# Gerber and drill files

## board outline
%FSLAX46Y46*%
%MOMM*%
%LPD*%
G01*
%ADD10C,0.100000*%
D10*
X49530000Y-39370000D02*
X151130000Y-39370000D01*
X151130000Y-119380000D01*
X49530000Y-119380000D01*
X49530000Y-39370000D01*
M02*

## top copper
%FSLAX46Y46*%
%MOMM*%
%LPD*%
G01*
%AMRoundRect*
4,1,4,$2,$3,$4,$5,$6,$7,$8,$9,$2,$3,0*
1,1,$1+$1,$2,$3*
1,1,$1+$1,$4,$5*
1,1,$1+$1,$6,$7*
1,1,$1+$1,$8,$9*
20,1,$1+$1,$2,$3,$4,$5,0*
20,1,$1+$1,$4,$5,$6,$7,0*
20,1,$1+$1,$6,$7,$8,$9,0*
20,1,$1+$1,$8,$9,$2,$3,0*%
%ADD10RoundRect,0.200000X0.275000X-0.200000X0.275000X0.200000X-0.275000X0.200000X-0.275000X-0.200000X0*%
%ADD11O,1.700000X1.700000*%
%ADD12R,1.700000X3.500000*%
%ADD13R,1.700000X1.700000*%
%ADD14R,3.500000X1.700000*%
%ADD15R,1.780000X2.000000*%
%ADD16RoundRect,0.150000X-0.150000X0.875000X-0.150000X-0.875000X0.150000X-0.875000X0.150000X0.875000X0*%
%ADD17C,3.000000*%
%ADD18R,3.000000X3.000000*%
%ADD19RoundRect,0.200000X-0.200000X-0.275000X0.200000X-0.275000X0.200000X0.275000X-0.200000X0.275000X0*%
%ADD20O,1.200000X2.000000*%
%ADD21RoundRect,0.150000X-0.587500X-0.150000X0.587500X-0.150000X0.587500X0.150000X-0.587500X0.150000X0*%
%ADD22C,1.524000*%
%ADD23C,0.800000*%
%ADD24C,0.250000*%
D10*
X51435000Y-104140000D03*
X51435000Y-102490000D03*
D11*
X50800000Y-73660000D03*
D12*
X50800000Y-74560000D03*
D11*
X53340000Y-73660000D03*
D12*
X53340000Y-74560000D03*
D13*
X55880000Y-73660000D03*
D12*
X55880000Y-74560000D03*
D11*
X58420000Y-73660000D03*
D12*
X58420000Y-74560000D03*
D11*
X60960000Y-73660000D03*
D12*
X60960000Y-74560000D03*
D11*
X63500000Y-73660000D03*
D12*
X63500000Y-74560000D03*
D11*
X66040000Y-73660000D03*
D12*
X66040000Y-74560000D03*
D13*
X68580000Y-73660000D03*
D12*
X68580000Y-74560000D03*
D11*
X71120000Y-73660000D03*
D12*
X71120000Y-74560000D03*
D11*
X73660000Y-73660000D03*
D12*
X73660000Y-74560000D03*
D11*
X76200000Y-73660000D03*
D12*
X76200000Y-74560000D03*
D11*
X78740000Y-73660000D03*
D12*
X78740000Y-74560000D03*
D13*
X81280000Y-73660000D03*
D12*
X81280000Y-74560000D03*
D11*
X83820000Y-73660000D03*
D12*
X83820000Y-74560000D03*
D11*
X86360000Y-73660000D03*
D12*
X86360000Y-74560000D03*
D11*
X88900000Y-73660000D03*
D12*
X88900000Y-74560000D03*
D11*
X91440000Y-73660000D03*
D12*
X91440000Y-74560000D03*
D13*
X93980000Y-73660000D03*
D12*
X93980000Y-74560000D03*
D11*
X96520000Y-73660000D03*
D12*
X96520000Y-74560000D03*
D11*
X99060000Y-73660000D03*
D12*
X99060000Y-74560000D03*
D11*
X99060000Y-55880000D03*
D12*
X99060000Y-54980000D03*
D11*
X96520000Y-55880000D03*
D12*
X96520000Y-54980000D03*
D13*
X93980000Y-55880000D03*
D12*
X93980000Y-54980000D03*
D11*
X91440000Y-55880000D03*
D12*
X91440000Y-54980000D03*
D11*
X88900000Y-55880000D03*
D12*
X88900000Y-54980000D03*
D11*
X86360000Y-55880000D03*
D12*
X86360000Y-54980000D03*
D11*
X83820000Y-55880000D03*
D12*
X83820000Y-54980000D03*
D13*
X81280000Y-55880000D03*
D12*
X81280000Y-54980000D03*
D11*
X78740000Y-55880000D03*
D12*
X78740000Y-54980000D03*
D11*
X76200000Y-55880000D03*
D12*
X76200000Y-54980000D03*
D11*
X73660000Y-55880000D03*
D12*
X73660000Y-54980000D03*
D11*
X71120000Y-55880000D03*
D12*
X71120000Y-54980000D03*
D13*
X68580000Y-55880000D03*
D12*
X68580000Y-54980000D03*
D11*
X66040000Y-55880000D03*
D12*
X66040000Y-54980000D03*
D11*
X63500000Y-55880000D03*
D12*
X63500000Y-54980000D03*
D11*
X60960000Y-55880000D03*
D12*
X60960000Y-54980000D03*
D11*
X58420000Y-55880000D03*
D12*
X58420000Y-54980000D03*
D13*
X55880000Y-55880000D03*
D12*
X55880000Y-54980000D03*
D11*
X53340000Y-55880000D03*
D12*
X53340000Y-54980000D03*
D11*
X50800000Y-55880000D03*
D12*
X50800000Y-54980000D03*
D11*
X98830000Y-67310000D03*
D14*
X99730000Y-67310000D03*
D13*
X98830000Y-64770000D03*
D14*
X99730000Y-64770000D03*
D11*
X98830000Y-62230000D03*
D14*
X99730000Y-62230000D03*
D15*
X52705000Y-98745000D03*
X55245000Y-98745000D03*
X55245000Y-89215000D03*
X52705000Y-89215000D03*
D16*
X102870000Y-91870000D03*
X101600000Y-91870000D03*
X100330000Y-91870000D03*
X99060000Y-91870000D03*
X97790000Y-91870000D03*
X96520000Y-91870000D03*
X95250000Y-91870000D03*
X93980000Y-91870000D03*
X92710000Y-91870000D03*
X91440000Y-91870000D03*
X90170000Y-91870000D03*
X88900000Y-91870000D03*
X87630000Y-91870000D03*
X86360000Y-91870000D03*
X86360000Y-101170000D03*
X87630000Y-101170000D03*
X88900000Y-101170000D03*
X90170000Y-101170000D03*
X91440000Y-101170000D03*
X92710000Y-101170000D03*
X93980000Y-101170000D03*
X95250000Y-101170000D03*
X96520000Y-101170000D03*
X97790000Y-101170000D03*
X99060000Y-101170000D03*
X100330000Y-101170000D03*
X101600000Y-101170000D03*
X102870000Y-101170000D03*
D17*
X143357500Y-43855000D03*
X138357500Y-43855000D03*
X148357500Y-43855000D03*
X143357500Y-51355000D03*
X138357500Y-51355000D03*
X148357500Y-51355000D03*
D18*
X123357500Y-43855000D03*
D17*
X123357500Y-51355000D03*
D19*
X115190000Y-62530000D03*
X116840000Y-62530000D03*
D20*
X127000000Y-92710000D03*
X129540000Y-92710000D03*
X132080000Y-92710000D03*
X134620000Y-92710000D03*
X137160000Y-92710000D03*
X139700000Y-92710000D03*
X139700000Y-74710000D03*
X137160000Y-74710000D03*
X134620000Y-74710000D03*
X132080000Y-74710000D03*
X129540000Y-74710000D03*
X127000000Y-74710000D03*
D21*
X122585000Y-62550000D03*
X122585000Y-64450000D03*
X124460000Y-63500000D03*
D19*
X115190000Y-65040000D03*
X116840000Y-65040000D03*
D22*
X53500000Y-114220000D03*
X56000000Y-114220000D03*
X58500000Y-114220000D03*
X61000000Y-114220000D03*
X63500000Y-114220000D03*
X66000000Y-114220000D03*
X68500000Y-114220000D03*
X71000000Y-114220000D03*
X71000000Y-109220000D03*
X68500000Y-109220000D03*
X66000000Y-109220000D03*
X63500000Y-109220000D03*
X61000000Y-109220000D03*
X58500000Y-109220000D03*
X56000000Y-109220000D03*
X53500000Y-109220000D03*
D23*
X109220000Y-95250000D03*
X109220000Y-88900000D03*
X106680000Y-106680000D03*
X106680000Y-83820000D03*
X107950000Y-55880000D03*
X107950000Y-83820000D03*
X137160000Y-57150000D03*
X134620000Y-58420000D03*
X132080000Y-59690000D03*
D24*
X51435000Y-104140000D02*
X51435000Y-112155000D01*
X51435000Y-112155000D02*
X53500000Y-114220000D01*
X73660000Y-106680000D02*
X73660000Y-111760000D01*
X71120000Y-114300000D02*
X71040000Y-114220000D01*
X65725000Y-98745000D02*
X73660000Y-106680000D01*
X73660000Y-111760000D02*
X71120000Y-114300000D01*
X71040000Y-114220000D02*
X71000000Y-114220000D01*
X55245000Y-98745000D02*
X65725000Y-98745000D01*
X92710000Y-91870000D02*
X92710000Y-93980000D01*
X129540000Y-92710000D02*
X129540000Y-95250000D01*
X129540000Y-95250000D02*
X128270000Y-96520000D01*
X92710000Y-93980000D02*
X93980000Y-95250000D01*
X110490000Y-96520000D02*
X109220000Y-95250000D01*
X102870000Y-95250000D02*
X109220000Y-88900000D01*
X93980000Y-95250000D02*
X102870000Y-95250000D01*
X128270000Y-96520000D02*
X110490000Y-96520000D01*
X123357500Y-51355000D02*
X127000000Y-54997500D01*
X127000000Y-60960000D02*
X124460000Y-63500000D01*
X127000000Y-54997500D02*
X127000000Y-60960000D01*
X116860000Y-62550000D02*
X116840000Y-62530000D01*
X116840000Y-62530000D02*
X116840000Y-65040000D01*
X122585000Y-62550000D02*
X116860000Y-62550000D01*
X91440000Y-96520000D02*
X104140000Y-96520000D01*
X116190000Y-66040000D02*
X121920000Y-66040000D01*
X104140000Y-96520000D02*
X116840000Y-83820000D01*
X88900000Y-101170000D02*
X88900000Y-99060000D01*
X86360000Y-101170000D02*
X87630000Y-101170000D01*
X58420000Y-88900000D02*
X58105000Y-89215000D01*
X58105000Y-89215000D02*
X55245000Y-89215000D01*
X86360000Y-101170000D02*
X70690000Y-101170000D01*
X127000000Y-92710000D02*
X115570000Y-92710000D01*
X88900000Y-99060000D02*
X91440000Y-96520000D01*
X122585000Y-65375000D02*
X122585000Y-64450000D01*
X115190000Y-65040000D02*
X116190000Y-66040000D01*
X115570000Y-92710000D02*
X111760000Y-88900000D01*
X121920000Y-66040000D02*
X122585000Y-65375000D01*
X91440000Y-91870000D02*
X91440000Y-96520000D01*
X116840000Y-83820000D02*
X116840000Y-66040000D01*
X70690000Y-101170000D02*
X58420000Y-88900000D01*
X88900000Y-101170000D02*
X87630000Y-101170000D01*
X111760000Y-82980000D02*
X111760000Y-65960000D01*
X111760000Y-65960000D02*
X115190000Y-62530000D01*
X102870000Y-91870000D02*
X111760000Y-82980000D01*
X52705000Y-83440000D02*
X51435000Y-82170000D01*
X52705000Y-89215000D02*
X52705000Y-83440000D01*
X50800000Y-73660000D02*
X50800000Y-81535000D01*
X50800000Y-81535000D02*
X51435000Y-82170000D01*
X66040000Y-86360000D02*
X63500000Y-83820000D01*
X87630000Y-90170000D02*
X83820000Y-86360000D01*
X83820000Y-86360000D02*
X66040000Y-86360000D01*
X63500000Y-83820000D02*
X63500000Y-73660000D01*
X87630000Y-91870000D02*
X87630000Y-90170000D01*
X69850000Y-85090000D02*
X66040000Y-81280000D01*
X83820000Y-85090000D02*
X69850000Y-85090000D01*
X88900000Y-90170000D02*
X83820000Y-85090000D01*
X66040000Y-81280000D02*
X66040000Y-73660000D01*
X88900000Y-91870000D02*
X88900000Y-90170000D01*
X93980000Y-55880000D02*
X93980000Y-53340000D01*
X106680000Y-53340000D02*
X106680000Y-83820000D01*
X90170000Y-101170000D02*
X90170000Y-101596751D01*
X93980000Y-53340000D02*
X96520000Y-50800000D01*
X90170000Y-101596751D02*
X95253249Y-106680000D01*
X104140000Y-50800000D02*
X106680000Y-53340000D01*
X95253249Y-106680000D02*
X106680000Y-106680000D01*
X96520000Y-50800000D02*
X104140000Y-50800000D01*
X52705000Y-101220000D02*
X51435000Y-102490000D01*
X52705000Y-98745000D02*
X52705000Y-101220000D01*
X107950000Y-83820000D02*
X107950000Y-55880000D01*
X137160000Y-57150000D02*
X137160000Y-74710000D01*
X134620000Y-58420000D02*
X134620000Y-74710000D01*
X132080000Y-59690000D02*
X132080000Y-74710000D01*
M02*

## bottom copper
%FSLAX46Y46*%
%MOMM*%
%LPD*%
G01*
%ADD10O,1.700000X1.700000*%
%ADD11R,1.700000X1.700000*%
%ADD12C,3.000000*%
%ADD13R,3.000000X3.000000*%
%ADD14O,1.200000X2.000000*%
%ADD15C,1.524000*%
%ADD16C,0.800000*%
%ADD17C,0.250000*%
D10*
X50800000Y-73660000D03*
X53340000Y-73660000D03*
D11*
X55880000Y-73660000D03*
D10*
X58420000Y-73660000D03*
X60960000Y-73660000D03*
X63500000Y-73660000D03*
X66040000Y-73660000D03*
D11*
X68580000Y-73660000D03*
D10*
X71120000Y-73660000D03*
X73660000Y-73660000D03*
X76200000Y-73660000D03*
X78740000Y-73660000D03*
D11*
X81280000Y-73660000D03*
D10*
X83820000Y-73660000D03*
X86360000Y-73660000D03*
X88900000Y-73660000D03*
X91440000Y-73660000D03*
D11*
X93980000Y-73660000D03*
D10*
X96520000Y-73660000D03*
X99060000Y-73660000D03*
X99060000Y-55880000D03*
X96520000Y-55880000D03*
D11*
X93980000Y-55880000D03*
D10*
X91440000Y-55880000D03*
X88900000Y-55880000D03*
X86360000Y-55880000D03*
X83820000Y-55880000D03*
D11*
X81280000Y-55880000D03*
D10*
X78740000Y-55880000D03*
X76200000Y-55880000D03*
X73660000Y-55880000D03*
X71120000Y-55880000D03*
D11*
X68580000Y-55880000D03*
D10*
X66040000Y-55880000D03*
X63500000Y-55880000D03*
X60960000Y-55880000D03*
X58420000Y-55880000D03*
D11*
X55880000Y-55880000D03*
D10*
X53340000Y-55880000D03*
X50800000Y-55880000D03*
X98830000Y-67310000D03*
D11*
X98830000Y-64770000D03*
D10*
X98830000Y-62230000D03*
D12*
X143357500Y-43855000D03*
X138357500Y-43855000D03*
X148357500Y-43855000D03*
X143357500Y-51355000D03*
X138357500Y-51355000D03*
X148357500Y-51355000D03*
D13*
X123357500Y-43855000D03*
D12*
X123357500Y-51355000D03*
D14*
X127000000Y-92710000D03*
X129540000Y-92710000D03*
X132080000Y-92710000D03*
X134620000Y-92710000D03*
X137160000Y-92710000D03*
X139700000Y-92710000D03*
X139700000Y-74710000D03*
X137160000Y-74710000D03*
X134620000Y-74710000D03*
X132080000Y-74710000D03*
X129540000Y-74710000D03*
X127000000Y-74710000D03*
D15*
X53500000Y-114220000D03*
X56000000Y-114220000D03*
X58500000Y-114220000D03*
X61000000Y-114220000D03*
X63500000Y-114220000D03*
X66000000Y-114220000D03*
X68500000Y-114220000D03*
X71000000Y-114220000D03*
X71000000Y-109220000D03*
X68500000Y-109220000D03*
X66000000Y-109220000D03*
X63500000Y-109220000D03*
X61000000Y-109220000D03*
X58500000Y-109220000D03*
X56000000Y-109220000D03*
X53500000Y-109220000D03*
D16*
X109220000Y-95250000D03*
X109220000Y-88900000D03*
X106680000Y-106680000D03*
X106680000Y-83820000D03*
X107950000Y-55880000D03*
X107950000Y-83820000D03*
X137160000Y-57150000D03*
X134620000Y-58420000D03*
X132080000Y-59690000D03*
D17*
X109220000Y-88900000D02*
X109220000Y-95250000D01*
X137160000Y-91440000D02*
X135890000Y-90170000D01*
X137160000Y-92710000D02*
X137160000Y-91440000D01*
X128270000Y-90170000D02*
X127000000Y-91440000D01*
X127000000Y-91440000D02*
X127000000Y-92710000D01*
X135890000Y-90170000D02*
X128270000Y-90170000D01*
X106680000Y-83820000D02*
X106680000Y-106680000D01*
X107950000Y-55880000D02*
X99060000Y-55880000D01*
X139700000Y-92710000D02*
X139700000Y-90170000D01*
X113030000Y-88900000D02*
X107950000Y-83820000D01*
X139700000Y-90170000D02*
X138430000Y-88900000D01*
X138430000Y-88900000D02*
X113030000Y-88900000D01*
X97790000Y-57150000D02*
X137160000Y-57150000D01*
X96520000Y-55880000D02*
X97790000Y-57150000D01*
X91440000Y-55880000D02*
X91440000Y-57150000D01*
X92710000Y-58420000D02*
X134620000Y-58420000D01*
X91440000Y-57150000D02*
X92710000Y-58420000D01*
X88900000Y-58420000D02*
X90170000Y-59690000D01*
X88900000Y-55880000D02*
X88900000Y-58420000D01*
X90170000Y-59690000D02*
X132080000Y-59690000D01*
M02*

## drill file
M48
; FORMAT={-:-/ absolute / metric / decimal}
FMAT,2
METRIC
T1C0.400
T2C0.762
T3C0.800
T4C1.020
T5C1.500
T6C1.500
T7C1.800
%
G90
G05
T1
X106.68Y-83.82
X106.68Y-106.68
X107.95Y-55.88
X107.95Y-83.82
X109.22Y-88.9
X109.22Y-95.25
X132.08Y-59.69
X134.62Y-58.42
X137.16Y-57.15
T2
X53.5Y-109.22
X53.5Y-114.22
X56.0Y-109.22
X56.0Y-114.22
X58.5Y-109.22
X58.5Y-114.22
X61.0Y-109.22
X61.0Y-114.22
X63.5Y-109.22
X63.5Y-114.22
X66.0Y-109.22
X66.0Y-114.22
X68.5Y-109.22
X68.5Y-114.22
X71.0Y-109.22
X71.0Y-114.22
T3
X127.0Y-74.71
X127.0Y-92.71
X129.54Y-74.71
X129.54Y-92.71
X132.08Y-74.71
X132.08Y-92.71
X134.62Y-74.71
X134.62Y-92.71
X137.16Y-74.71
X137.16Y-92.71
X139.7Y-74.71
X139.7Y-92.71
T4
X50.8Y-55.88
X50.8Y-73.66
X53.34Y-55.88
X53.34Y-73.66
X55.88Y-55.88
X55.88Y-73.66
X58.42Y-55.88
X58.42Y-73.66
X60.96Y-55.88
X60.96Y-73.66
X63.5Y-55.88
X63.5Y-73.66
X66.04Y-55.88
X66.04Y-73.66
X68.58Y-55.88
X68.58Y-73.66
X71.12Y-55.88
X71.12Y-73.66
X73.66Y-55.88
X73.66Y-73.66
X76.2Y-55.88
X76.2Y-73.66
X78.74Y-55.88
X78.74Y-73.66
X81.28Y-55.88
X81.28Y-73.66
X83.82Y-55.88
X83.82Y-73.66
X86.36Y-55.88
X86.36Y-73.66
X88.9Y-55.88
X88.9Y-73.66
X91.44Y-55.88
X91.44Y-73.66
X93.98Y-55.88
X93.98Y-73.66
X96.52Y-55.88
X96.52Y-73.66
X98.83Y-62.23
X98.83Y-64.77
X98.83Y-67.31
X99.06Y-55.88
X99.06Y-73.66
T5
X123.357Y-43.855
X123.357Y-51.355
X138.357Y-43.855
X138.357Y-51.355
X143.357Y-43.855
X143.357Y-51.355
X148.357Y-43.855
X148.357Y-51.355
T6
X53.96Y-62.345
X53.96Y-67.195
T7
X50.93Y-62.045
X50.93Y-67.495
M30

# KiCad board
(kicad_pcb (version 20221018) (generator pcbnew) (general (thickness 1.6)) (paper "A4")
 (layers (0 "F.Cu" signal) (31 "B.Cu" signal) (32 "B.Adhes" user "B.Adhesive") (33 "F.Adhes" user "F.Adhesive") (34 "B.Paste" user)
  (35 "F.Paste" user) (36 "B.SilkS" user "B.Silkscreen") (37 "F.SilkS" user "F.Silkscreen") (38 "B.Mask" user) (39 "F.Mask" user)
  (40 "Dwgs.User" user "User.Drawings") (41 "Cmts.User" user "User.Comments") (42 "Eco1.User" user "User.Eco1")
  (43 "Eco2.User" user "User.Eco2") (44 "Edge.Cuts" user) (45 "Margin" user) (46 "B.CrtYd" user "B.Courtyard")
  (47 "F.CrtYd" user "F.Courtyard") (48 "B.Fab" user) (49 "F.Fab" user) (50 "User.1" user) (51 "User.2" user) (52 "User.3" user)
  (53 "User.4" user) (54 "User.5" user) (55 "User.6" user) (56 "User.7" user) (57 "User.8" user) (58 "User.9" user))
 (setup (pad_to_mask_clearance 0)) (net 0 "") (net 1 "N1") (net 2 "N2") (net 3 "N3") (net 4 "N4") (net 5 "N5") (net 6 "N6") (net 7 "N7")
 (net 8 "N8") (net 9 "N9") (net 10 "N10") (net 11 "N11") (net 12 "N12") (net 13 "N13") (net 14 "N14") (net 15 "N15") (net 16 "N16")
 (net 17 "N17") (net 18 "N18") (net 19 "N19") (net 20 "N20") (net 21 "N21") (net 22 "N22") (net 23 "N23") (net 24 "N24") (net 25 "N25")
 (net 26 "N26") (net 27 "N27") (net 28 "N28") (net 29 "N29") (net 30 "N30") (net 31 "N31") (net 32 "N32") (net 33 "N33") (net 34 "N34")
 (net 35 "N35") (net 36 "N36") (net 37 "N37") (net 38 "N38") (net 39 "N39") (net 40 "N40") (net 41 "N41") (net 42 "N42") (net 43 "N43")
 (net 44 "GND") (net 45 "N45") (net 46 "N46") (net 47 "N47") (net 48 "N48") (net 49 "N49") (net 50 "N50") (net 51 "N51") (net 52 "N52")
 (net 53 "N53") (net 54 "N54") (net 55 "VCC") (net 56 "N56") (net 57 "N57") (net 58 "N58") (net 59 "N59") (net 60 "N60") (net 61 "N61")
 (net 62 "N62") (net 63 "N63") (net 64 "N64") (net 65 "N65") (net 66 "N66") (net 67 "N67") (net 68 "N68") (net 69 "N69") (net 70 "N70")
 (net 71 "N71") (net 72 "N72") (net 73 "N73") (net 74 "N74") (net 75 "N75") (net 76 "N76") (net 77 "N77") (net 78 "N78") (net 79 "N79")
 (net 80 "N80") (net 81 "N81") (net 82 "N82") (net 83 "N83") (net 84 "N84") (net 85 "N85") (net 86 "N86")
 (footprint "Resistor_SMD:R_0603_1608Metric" (layer "F.Cu") (at 51.435 103.315 90)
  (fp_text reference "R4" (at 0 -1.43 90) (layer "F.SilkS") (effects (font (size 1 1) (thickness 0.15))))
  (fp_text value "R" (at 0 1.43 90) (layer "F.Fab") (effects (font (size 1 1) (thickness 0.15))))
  (pad "1" smd roundrect (at -0.825 0 90) (size 0.8 0.95) (layers "F.Cu" "F.Paste" "F.Mask") (roundrect_rratio 0.25) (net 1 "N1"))
  (pad "2" smd roundrect (at 0.825 0 90) (size 0.8 0.95) (layers "F.Cu" "F.Paste" "F.Mask") (roundrect_rratio 0.25) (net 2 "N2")))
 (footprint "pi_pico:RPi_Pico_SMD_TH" (layer "F.Cu") (at 74.93 64.77 90)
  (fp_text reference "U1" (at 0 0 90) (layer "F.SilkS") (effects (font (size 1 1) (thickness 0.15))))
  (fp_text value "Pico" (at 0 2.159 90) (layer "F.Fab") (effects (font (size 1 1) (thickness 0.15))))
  (pad "" np_thru_hole oval (at -2.725 -24 90) (size 1.8 1.8) (drill 1.8) (layers "*.Cu" "*.Mask"))
  (pad "" np_thru_hole oval (at -2.425 -20.97 90) (size 1.5 1.5) (drill 1.5) (layers "*.Cu" "*.Mask"))
  (pad "" np_thru_hole oval (at 2.425 -20.97 90) (size 1.5 1.5) (drill 1.5) (layers "*.Cu" "*.Mask"))
  (pad "" np_thru_hole oval (at 2.725 -24 90) (size 1.8 1.8) (drill 1.8) (layers "*.Cu" "*.Mask"))
  (pad "1" thru_hole oval (at -8.89 -24.13 90) (size 1.7 1.7) (drill 1.02) (layers "*.Cu" "*.Mask") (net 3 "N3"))
  (pad "1" smd rect (at -8.89 -24.13 90) (size 3.5 1.7) (drill (offset -0.9 0)) (layers "F.Cu" "F.Mask") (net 3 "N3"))
  (pad "2" thru_hole oval (at -8.89 -21.59 90) (size 1.7 1.7) (drill 1.02) (layers "*.Cu" "*.Mask") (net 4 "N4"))
  (pad "2" smd rect (at -8.89 -21.59 90) (size 3.5 1.7) (drill (offset -0.9 0)) (layers "F.Cu" "F.Mask") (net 4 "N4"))
  (pad "3" thru_hole rect (at -8.89 -19.05 90) (size 1.7 1.7) (drill 1.02) (layers "*.Cu" "*.Mask") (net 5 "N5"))
  (pad "3" smd rect (at -8.89 -19.05 90) (size 3.5 1.7) (drill (offset -0.9 0)) (layers "F.Cu" "F.Mask") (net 5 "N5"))
  (pad "4" thru_hole oval (at -8.89 -16.51 90) (size 1.7 1.7) (drill 1.02) (layers "*.Cu" "*.Mask") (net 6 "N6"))
  (pad "4" smd rect (at -8.89 -16.51 90) (size 3.5 1.7) (drill (offset -0.9 0)) (layers "F.Cu" "F.Mask") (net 6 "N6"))
  (pad "5" thru_hole oval (at -8.89 -13.97 90) (size 1.7 1.7) (drill 1.02) (layers "*.Cu" "*.Mask") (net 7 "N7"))
  (pad "5" smd rect (at -8.89 -13.97 90) (size 3.5 1.7) (drill (offset -0.9 0)) (layers "F.Cu" "F.Mask") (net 7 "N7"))
  (pad "6" thru_hole oval (at -8.89 -11.43 90) (size 1.7 1.7) (drill 1.02) (layers "*.Cu" "*.Mask") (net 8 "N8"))
  (pad "6" smd rect (at -8.89 -11.43 90) (size 3.5 1.7) (drill (offset -0.9 0)) (layers "F.Cu" "F.Mask") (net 8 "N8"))
  (pad "7" thru_hole oval (at -8.89 -8.89 90) (size 1.7 1.7) (drill 1.02) (layers "*.Cu" "*.Mask") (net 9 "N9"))
  (pad "7" smd rect (at -8.89 -8.89 90) (size 3.5 1.7) (drill (offset -0.9 0)) (layers "F.Cu" "F.Mask") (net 9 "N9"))
  (pad "8" thru_hole rect (at -8.89 -6.35 90) (size 1.7 1.7) (drill 1.02) (layers "*.Cu" "*.Mask") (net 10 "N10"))
  (pad "8" smd rect (at -8.89 -6.35 90) (size 3.5 1.7) (drill (offset -0.9 0)) (layers "F.Cu" "F.Mask") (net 10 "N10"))
  (pad "9" thru_hole oval (at -8.89 -3.81 90) (size 1.7 1.7) (drill 1.02) (layers "*.Cu" "*.Mask") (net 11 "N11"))
  (pad "9" smd rect (at -8.89 -3.81 90) (size 3.5 1.7) (drill (offset -0.9 0)) (layers "F.Cu" "F.Mask") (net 11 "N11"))
  (pad "10" thru_hole oval (at -8.89 -1.27 90) (size 1.7 1.7) (drill 1.02) (layers "*.Cu" "*.Mask") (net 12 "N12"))
  (pad "10" smd rect (at -8.89 -1.27 90) (size 3.5 1.7) (drill (offset -0.9 0)) (layers "F.Cu" "F.Mask") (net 12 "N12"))
  (pad "11" thru_hole oval (at -8.89 1.27 90) (size 1.7 1.7) (drill 1.02) (layers "*.Cu" "*.Mask") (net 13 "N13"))
  (pad "11" smd rect (at -8.89 1.27 90) (size 3.5 1.7) (drill (offset -0.9 0)) (layers "F.Cu" "F.Mask") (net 13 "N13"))
  (pad "12" thru_hole oval (at -8.89 3.81 90) (size 1.7 1.7) (drill 1.02) (layers "*.Cu" "*.Mask") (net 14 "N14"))
  (pad "12" smd rect (at -8.89 3.81 90) (size 3.5 1.7) (drill (offset -0.9 0)) (layers "F.Cu" "F.Mask") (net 14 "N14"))
  (pad "13" thru_hole rect (at -8.89 6.35 90) (size 1.7 1.7) (drill 1.02) (layers "*.Cu" "*.Mask") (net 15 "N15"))
  (pad "13" smd rect (at -8.89 6.35 90) (size 3.5 1.7) (drill (offset -0.9 0)) (layers "F.Cu" "F.Mask") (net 15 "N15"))
  (pad "14" thru_hole oval (at -8.89 8.89 90) (size 1.7 1.7) (drill 1.02) (layers "*.Cu" "*.Mask") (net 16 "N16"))
  (pad "14" smd rect (at -8.89 8.89 90) (size 3.5 1.7) (drill (offset -0.9 0)) (layers "F.Cu" "F.Mask") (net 16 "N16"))
  (pad "15" thru_hole oval (at -8.89 11.43 90) (size 1.7 1.7) (drill 1.02) (layers "*.Cu" "*.Mask") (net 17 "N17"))
  (pad "15" smd rect (at -8.89 11.43 90) (size 3.5 1.7) (drill (offset -0.9 0)) (layers "F.Cu" "F.Mask") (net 17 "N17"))
  (pad "16" thru_hole oval (at -8.89 13.97 90) (size 1.7 1.7) (drill 1.02) (layers "*.Cu" "*.Mask") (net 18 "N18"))
  (pad "16" smd rect (at -8.89 13.97 90) (size 3.5 1.7) (drill (offset -0.9 0)) (layers "F.Cu" "F.Mask") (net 18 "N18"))
  (pad "17" thru_hole oval (at -8.89 16.51 90) (size 1.7 1.7) (drill 1.02) (layers "*.Cu" "*.Mask") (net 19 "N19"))
  (pad "17" smd rect (at -8.89 16.51 90) (size 3.5 1.7) (drill (offset -0.9 0)) (layers "F.Cu" "F.Mask") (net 19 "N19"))
  (pad "18" thru_hole rect (at -8.89 19.05 90) (size 1.7 1.7) (drill 1.02) (layers "*.Cu" "*.Mask") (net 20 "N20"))
  (pad "18" smd rect (at -8.89 19.05 90) (size 3.5 1.7) (drill (offset -0.9 0)) (layers "F.Cu" "F.Mask") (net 20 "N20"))
  (pad "19" thru_hole oval (at -8.89 21.59 90) (size 1.7 1.7) (drill 1.02) (layers "*.Cu" "*.Mask") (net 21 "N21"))
  (pad "19" smd rect (at -8.89 21.59 90) (size 3.5 1.7) (drill (offset -0.9 0)) (layers "F.Cu" "F.Mask") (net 21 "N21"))
  (pad "20" thru_hole oval (at -8.89 24.13 90) (size 1.7 1.7) (drill 1.02) (layers "*.Cu" "*.Mask") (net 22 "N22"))
  (pad "20" smd rect (at -8.89 24.13 90) (size 3.5 1.7) (drill (offset -0.9 0)) (layers "F.Cu" "F.Mask") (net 22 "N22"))
  (pad "21" thru_hole oval (at 8.89 24.13 90) (size 1.7 1.7) (drill 1.02) (layers "*.Cu" "*.Mask") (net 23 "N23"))
  (pad "21" smd rect (at 8.89 24.13 90) (size 3.5 1.7) (drill (offset 0.9 0)) (layers "F.Cu" "F.Mask") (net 23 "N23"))
  (pad "22" thru_hole oval (at 8.89 21.59 90) (size 1.7 1.7) (drill 1.02) (layers "*.Cu" "*.Mask") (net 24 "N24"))
  (pad "22" smd rect (at 8.89 21.59 90) (size 3.5 1.7) (drill (offset 0.9 0)) (layers "F.Cu" "F.Mask") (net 24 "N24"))
  (pad "23" thru_hole rect (at 8.89 19.05 90) (size 1.7 1.7) (drill 1.02) (layers "*.Cu" "*.Mask") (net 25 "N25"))
  (pad "23" smd rect (at 8.89 19.05 90) (size 3.5 1.7) (drill (offset 0.9 0)) (layers "F.Cu" "F.Mask") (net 25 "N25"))
  (pad "24" thru_hole oval (at 8.89 16.51 90) (size 1.7 1.7) (drill 1.02) (layers "*.Cu" "*.Mask") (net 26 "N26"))
  (pad "24" smd rect (at 8.89 16.51 90) (size 3.5 1.7) (drill (offset 0.9 0)) (layers "F.Cu" "F.Mask") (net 26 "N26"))
  (pad "25" thru_hole oval (at 8.89 13.97 90) (size 1.7 1.7) (drill 1.02) (layers "*.Cu" "*.Mask") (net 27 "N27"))
  (pad "25" smd rect (at 8.89 13.97 90) (size 3.5 1.7) (drill (offset 0.9 0)) (layers "F.Cu" "F.Mask") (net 27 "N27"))
  (pad "26" thru_hole oval (at 8.89 11.43 90) (size 1.7 1.7) (drill 1.02) (layers "*.Cu" "*.Mask") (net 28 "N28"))
  (pad "26" smd rect (at 8.89 11.43 90) (size 3.5 1.7) (drill (offset 0.9 0)) (layers "F.Cu" "F.Mask") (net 28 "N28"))
  (pad "27" thru_hole oval (at 8.89 8.89 90) (size 1.7 1.7) (drill 1.02) (layers "*.Cu" "*.Mask") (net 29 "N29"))
  (pad "27" smd rect (at 8.89 8.89 90) (size 3.5 1.7) (drill (offset 0.9 0)) (layers "F.Cu" "F.Mask") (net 29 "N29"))
  (pad "28" thru_hole rect (at 8.89 6.35 90) (size 1.7 1.7) (drill 1.02) (layers "*.Cu" "*.Mask") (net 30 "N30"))
  (pad "28" smd rect (at 8.89 6.35 90) (size 3.5 1.7) (drill (offset 0.9 0)) (layers "F.Cu" "F.Mask") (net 30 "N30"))
  (pad "29" thru_hole oval (at 8.89 3.81 90) (size 1.7 1.7) (drill 1.02) (layers "*.Cu" "*.Mask") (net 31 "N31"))
  (pad "29" smd rect (at 8.89 3.81 90) (size 3.5 1.7) (drill (offset 0.9 0)) (layers "F.Cu" "F.Mask") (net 31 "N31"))
  (pad "30" thru_hole oval (at 8.89 1.27 90) (size 1.7 1.7) (drill 1.02) (layers "*.Cu" "*.Mask") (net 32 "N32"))
  (pad "30" smd rect (at 8.89 1.27 90) (size 3.5 1.7) (drill (offset 0.9 0)) (layers "F.Cu" "F.Mask") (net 32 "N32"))
  (pad "31" thru_hole oval (at 8.89 -1.27 90) (size 1.7 1.7) (drill 1.02) (layers "*.Cu" "*.Mask") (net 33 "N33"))
  (pad "31" smd rect (at 8.89 -1.27 90) (size 3.5 1.7) (drill (offset 0.9 0)) (layers "F.Cu" "F.Mask") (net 33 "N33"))
  (pad "32" thru_hole oval (at 8.89 -3.81 90) (size 1.7 1.7) (drill 1.02) (layers "*.Cu" "*.Mask") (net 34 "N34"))
  (pad "32" smd rect (at 8.89 -3.81 90) (size 3.5 1.7) (drill (offset 0.9 0)) (layers "F.Cu" "F.Mask") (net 34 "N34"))
  (pad "33" thru_hole rect (at 8.89 -6.35 90) (size 1.7 1.7) (drill 1.02) (layers "*.Cu" "*.Mask") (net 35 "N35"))
  (pad "33" smd rect (at 8.89 -6.35 90) (size 3.5 1.7) (drill (offset 0.9 0)) (layers "F.Cu" "F.Mask") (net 35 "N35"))
  (pad "34" thru_hole oval (at 8.89 -8.89 90) (size 1.7 1.7) (drill 1.02) (layers "*.Cu" "*.Mask") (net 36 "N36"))
  (pad "34" smd rect (at 8.89 -8.89 90) (size 3.5 1.7) (drill (offset 0.9 0)) (layers "F.Cu" "F.Mask") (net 36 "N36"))
  (pad "35" thru_hole oval (at 8.89 -11.43 90) (size 1.7 1.7) (drill 1.02) (layers "*.Cu" "*.Mask") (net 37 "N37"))
  (pad "35" smd rect (at 8.89 -11.43 90) (size 3.5 1.7) (drill (offset 0.9 0)) (layers "F.Cu" "F.Mask") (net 37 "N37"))
  (pad "36" thru_hole oval (at 8.89 -13.97 90) (size 1.7 1.7) (drill 1.02) (layers "*.Cu" "*.Mask") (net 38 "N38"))
  (pad "36" smd rect (at 8.89 -13.97 90) (size 3.5 1.7) (drill (offset 0.9 0)) (layers "F.Cu" "F.Mask") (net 38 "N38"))
  (pad "37" thru_hole oval (at 8.89 -16.51 90) (size 1.7 1.7) (drill 1.02) (layers "*.Cu" "*.Mask") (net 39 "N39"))
  (pad "37" smd rect (at 8.89 -16.51 90) (size 3.5 1.7) (drill (offset 0.9 0)) (layers "F.Cu" "F.Mask") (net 39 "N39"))
  (pad "38" thru_hole rect (at 8.89 -19.05 90) (size 1.7 1.7) (drill 1.02) (layers "*.Cu" "*.Mask") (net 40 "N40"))
  (pad "38" smd rect (at 8.89 -19.05 90) (size 3.5 1.7) (drill (offset 0.9 0)) (layers "F.Cu" "F.Mask") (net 40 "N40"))
  (pad "39" thru_hole oval (at 8.89 -21.59 90) (size 1.7 1.7) (drill 1.02) (layers "*.Cu" "*.Mask") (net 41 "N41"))
  (pad "39" smd rect (at 8.89 -21.59 90) (size 3.5 1.7) (drill (offset 0.9 0)) (layers "F.Cu" "F.Mask") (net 41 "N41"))
  (pad "40" thru_hole oval (at 8.89 -24.13 90) (size 1.7 1.7) (drill 1.02) (layers "*.Cu" "*.Mask") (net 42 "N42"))
  (pad "40" smd rect (at 8.89 -24.13 90) (size 3.5 1.7) (drill (offset 0.9 0)) (layers "F.Cu" "F.Mask") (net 42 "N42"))
  (pad "41" thru_hole oval (at -2.54 23.9 90) (size 1.7 1.7) (drill 1.02) (layers "*.Cu" "*.Mask") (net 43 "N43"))
  (pad "41" smd rect (at -2.54 23.9 180) (size 3.5 1.7) (drill (offset -0.9 0)) (layers "F.Cu" "F.Mask") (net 43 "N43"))
  (pad "42" thru_hole rect (at 0 23.9 90) (size 1.7 1.7) (drill 1.02) (layers "*.Cu" "*.Mask") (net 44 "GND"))
  (pad "42" smd rect (at 0 23.9 180) (size 3.5 1.7) (drill (offset -0.9 0)) (layers "F.Cu" "F.Mask") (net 44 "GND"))
  (pad "43" thru_hole oval (at 2.54 23.9 90) (size 1.7 1.7) (drill 1.02) (layers "*.Cu" "*.Mask") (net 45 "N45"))
  (pad "43" smd rect (at 2.54 23.9 180) (size 3.5 1.7) (drill (offset -0.9 0)) (layers "F.Cu" "F.Mask") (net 45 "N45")))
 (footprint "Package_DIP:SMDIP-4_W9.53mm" (layer "F.Cu") (at 53.975 93.98 90)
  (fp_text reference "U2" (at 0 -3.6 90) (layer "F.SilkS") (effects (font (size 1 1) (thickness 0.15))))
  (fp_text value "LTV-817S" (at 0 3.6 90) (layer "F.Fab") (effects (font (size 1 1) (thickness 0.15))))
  (pad "1" smd rect (at -4.765 -1.27 90) (size 2 1.78) (layers "F.Cu" "F.Paste" "F.Mask") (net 2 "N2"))
  (pad "2" smd rect (at -4.765 1.27 90) (size 2 1.78) (layers "F.Cu" "F.Paste" "F.Mask") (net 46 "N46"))
  (pad "3" smd rect (at 4.765 1.27 90) (size 2 1.78) (layers "F.Cu" "F.Paste" "F.Mask") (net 44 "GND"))
  (pad "4" smd rect (at 4.765 -1.27 90) (size 2 1.78) (layers "F.Cu" "F.Paste" "F.Mask") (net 3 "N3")))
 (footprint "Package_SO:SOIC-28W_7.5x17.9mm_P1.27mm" (layer "F.Cu") (at 94.615 96.52 -90)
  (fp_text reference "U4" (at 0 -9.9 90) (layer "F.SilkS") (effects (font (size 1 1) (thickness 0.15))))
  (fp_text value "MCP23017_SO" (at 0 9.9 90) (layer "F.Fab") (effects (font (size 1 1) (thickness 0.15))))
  (pad "1" smd roundrect (at -4.65 -8.255 270) (size 2.05 0.6) (layers "F.Cu" "F.Paste" "F.Mask") (roundrect_rratio 0.25) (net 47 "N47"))
  (pad "2" smd roundrect (at -4.65 -6.985 270) (size 2.05 0.6) (layers "F.Cu" "F.Paste" "F.Mask") (roundrect_rratio 0.25) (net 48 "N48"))
  (pad "3" smd roundrect (at -4.65 -5.715 270) (size 2.05 0.6) (layers "F.Cu" "F.Paste" "F.Mask") (roundrect_rratio 0.25) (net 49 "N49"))
  (pad "4" smd roundrect (at -4.65 -4.445 270) (size 2.05 0.6) (layers "F.Cu" "F.Paste" "F.Mask") (roundrect_rratio 0.25) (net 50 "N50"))
  (pad "5" smd roundrect (at -4.65 -3.175 270) (size 2.05 0.6) (layers "F.Cu" "F.Paste" "F.Mask") (roundrect_rratio 0.25) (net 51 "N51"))
  (pad "6" smd roundrect (at -4.65 -1.905 270) (size 2.05 0.6) (layers "F.Cu" "F.Paste" "F.Mask") (roundrect_rratio 0.25) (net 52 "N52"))
  (pad "7" smd roundrect (at -4.65 -0.635 270) (size 2.05 0.6) (layers "F.Cu" "F.Paste" "F.Mask") (roundrect_rratio 0.25) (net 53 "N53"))
  (pad "8" smd roundrect (at -4.65 0.635 270) (size 2.05 0.6) (layers "F.Cu" "F.Paste" "F.Mask") (roundrect_rratio 0.25) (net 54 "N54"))
  (pad "9" smd roundrect (at -4.65 1.905 270) (size 2.05 0.6) (layers "F.Cu" "F.Paste" "F.Mask") (roundrect_rratio 0.25) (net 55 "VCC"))
  (pad "10" smd roundrect (at -4.65 3.175 270) (size 2.05 0.6) (layers "F.Cu" "F.Paste" "F.Mask") (roundrect_rratio 0.25) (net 44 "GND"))
  (pad "11" smd roundrect (at -4.65 4.445 270) (size 2.05 0.6) (layers "F.Cu" "F.Paste" "F.Mask") (roundrect_rratio 0.25) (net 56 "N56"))
  (pad "12" smd roundrect (at -4.65 5.715 270) (size 2.05 0.6) (layers "F.Cu" "F.Paste" "F.Mask") (roundrect_rratio 0.25) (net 9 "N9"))
  (pad "13" smd roundrect (at -4.65 6.985 270) (size 2.05 0.6) (layers "F.Cu" "F.Paste" "F.Mask") (roundrect_rratio 0.25) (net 8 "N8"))
  (pad "14" smd roundrect (at -4.65 8.255 270) (size 2.05 0.6) (layers "F.Cu" "F.Paste" "F.Mask") (roundrect_rratio 0.25) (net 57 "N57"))
  (pad "15" smd roundrect (at 4.65 8.255 270) (size 2.05 0.6) (layers "F.Cu" "F.Paste" "F.Mask") (roundrect_rratio 0.25) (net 44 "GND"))
  (pad "16" smd roundrect (at 4.65 6.985 270) (size 2.05 0.6) (layers "F.Cu" "F.Paste" "F.Mask") (roundrect_rratio 0.25) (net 44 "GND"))
  (pad "17" smd roundrect (at 4.65 5.715 270) (size 2.05 0.6) (layers "F.Cu" "F.Paste" "F.Mask") (roundrect_rratio 0.25) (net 44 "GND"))
  (pad "18" smd roundrect (at 4.65 4.445 270) (size 2.05 0.6) (layers "F.Cu" "F.Paste" "F.Mask") (roundrect_rratio 0.25) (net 25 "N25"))
  (pad "19" smd roundrect (at 4.65 3.175 270) (size 2.05 0.6) (layers "F.Cu" "F.Paste" "F.Mask") (roundrect_rratio 0.25) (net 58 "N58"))
  (pad "20" smd roundrect (at 4.65 1.905 270) (size 2.05 0.6) (layers "F.Cu" "F.Paste" "F.Mask") (roundrect_rratio 0.25) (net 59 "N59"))
  (pad "21" smd roundrect (at 4.65 0.635 270) (size 2.05 0.6) (layers "F.Cu" "F.Paste" "F.Mask") (roundrect_rratio 0.25) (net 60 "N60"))
  (pad "22" smd roundrect (at 4.65 -0.635 270) (size 2.05 0.6) (layers "F.Cu" "F.Paste" "F.Mask") (roundrect_rratio 0.25) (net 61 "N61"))
  (pad "23" smd roundrect (at 4.65 -1.905 270) (size 2.05 0.6) (layers "F.Cu" "F.Paste" "F.Mask") (roundrect_rratio 0.25) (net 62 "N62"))
  (pad "24" smd roundrect (at 4.65 -3.175 270) (size 2.05 0.6) (layers "F.Cu" "F.Paste" "F.Mask") (roundrect_rratio 0.25) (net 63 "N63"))
  (pad "25" smd roundrect (at 4.65 -4.445 270) (size 2.05 0.6) (layers "F.Cu" "F.Paste" "F.Mask") (roundrect_rratio 0.25) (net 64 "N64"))
  (pad "26" smd roundrect (at 4.65 -5.715 270) (size 2.05 0.6) (layers "F.Cu" "F.Paste" "F.Mask") (roundrect_rratio 0.25) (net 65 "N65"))
  (pad "27" smd roundrect (at 4.65 -6.985 270) (size 2.05 0.6) (layers "F.Cu" "F.Paste" "F.Mask") (roundrect_rratio 0.25) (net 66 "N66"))
  (pad "28" smd roundrect (at 4.65 -8.255 270) (size 2.05 0.6) (layers "F.Cu" "F.Paste" "F.Mask") (roundrect_rratio 0.25) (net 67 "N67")))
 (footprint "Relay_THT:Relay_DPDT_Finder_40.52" (layer "F.Cu") (at 123.3575 43.855)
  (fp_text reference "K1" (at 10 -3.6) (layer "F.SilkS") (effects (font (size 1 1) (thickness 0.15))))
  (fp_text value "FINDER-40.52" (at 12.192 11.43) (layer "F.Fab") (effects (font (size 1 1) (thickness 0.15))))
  (pad "11" thru_hole circle (at 20 0) (size 3 3) (drill 1.5) (layers "*.Cu" "*.Mask") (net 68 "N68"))
  (pad "12" thru_hole circle (at 15 0) (size 3 3) (drill 1.5) (layers "*.Cu" "*.Mask") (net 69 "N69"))
  (pad "14" thru_hole circle (at 25 0) (size 3 3) (drill 1.5) (layers "*.Cu" "*.Mask") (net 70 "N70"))
  (pad "21" thru_hole circle (at 20 7.5) (size 3 3) (drill 1.5) (layers "*.Cu" "*.Mask") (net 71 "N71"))
  (pad "22" thru_hole circle (at 15 7.5) (size 3 3) (drill 1.5) (layers "*.Cu" "*.Mask") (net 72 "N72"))
  (pad "24" thru_hole circle (at 25 7.5) (size 3 3) (drill 1.5) (layers "*.Cu" "*.Mask") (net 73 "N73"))
  (pad "A1" thru_hole rect (at 0 0) (size 3 3) (drill 1.5) (layers "*.Cu" "*.Mask") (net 55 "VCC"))
  (pad "A2" thru_hole circle (at 0 7.5) (size 3 3) (drill 1.5) (layers "*.Cu" "*.Mask") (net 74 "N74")))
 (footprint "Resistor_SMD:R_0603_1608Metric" (layer "F.Cu") (at 116.015 62.53)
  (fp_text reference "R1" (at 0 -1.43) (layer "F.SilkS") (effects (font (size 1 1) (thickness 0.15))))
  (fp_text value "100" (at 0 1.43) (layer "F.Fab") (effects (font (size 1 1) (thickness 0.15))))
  (pad "1" smd roundrect (at -0.825 0) (size 0.8 0.95) (layers "F.Cu" "F.Paste" "F.Mask") (roundrect_rratio 0.25) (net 47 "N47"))
  (pad "2" smd roundrect (at 0.825 0) (size 0.8 0.95) (layers "F.Cu" "F.Paste" "F.Mask") (roundrect_rratio 0.25) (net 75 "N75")))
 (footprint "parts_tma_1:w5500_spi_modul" (layer "F.Cu") (at 133.35 83.71)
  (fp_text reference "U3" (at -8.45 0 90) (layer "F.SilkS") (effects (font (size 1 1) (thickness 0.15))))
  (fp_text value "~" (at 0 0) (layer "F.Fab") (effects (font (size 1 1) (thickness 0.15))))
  (pad "1" thru_hole oval (at -6.35 9) (size 1.2 2) (drill 0.8) (layers "*.Cu" "*.Mask") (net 44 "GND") (thermal_bridge_angle 45))
  (pad "2" thru_hole oval (at -3.81 9) (size 1.2 2) (drill 0.8) (layers "*.Cu" "*.Mask") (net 55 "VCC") (thermal_bridge_angle 45))
  (pad "3" thru_hole oval (at -1.27 9) (size 1.2 2) (drill 0.8) (layers "*.Cu" "*.Mask") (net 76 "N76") (thermal_bridge_angle 45))
  (pad "4" thru_hole oval (at 1.27 9) (size 1.2 2) (drill 0.8) (layers "*.Cu" "*.Mask") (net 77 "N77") (thermal_bridge_angle 45))
  (pad "5" thru_hole oval (at 3.81 9) (size 1.2 2) (drill 0.8) (layers "*.Cu" "*.Mask") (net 44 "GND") (thermal_bridge_angle 45))
  (pad "6" thru_hole oval (at 6.35 9) (size 1.2 2) (drill 0.8) (layers "*.Cu" "*.Mask") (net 23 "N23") (thermal_bridge_angle 45))
  (pad "7" thru_hole oval (at 6.35 -9) (size 1.2 2) (drill 0.8) (layers "*.Cu" "*.Mask") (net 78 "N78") (thermal_bridge_angle 45))
  (pad "8" thru_hole oval (at 3.81 -9) (size 1.2 2) (drill 0.8) (layers "*.Cu" "*.Mask") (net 24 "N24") (thermal_bridge_angle 45))
  (pad "9" thru_hole oval (at 1.27 -9) (size 1.2 2) (drill 0.8) (layers "*.Cu" "*.Mask") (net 26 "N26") (thermal_bridge_angle 45))
  (pad "10" thru_hole oval (at -1.27 -9) (size 1.2 2) (drill 0.8) (layers "*.Cu" "*.Mask") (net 27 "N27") (thermal_bridge_angle 45))
  (pad "11" thru_hole oval (at -3.81 -9) (size 1.2 2) (drill 0.8) (layers "*.Cu" "*.Mask") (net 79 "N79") (thermal_bridge_angle 45))
  (pad "12" thru_hole oval (at -6.35 -9) (size 1.2 2) (drill 0.8) (layers "*.Cu" "*.Mask") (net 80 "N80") (thermal_bridge_angle 45)))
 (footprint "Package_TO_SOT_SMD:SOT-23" (layer "F.Cu") (at 123.5225 63.5)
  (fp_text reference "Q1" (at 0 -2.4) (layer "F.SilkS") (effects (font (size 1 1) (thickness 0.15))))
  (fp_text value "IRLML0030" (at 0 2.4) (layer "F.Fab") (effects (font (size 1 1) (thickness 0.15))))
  (pad "1" smd roundrect (at -0.9375 -0.95) (size 1.475 0.6) (layers "F.Cu" "F.Paste" "F.Mask") (roundrect_rratio 0.25) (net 75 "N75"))
  (pad "2" smd roundrect (at -0.9375 0.95) (size 1.475 0.6) (layers "F.Cu" "F.Paste" "F.Mask") (roundrect_rratio 0.25) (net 44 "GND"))
  (pad "3" smd roundrect (at 0.9375 0) (size 1.475 0.6) (layers "F.Cu" "F.Paste" "F.Mask") (roundrect_rratio 0.25) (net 74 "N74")))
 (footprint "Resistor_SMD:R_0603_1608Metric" (layer "F.Cu") (at 116.015 65.04)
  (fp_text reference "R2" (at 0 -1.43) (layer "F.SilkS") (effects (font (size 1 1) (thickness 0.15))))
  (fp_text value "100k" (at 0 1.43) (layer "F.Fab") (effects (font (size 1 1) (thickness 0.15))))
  (pad "1" smd roundrect (at -0.825 0) (size 0.8 0.95) (layers "F.Cu" "F.Paste" "F.Mask") (roundrect_rratio 0.25) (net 44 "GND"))
  (pad "2" smd roundrect (at 0.825 0) (size 0.8 0.95) (layers "F.Cu" "F.Paste" "F.Mask") (roundrect_rratio 0.25) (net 75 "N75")))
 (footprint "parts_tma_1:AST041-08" (layer "F.Cu") (at 53.5 114.22 90)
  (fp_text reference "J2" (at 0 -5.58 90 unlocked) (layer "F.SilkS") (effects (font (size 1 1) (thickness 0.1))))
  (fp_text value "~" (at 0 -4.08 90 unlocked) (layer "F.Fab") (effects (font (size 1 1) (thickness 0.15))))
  (pad "1" thru_hole circle (at 0 0 90) (size 1.524 1.524) (drill 0.762) (layers "*.Cu" "*.Mask") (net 1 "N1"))
  (pad "2" thru_hole circle (at 0 2.5 90) (size 1.524 1.524) (drill 0.762) (layers "*.Cu" "*.Mask") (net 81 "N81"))
  (pad "3" thru_hole circle (at 0 5 90) (size 1.524 1.524) (drill 0.762) (layers "*.Cu" "*.Mask") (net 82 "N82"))
  (pad "4" thru_hole circle (at 0 7.5 90) (size 1.524 1.524) (drill 0.762) (layers "*.Cu" "*.Mask") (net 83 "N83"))
  (pad "5" thru_hole circle (at 0 10 90) (size 1.524 1.524) (drill 0.762) (layers "*.Cu" "*.Mask") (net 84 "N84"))
  (pad "6" thru_hole circle (at 0 12.5 90) (size 1.524 1.524) (drill 0.762) (layers "*.Cu" "*.Mask") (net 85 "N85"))
  (pad "7" thru_hole circle (at 0 15 90) (size 1.524 1.524) (drill 0.762) (layers "*.Cu" "*.Mask") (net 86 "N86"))
  (pad "8" thru_hole circle (at 0 17.5 90) (size 1.524 1.524) (drill 0.762) (layers "*.Cu" "*.Mask") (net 46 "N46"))
  (pad "9" thru_hole circle (at 5 17.5 90) (size 1.524 1.524) (drill 0.762) (layers "*.Cu" "*.Mask"))
  (pad "10" thru_hole circle (at 5 15 90) (size 1.524 1.524) (drill 0.762) (layers "*.Cu" "*.Mask"))
  (pad "11" thru_hole circle (at 5 12.5 90) (size 1.524 1.524) (drill 0.762) (layers "*.Cu" "*.Mask"))
  (pad "12" thru_hole circle (at 5 10 90) (size 1.524 1.524) (drill 0.762) (layers "*.Cu" "*.Mask"))
  (pad "13" thru_hole circle (at 5 7.5 90) (size 1.524 1.524) (drill 0.762) (layers "*.Cu" "*.Mask"))
  (pad "14" thru_hole circle (at 5 5 90) (size 1.524 1.524) (drill 0.762) (layers "*.Cu" "*.Mask"))
  (pad "15" thru_hole circle (at 5 2.5 90) (size 1.524 1.524) (drill 0.762) (layers "*.Cu" "*.Mask"))
  (pad "16" thru_hole circle (at 5 0 90) (size 1.524 1.524) (drill 0.762) (layers "*.Cu" "*.Mask")))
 (gr_rect (start 49.53 39.37) (end 151.13 119.38) (stroke (width 0.1) (type default)) (fill none) (layer "Edge.Cuts"))
 (segment (start 51.435 104.14) (end 51.435 112.155) (width 0.25) (layer "F.Cu") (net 1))
 (segment (start 51.435 112.155) (end 53.5 114.22) (width 0.25) (layer "F.Cu") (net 1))
 (segment (start 73.66 106.68) (end 73.66 111.76) (width 0.25) (layer "F.Cu") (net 46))
 (segment (start 71.12 114.3) (end 71.04 114.22) (width 0.25) (layer "F.Cu") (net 46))
 (segment (start 65.725 98.745) (end 73.66 106.68) (width 0.25) (layer "F.Cu") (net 46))
 (segment (start 73.66 111.76) (end 71.12 114.3) (width 0.25) (layer "F.Cu") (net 46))
 (segment (start 71.04 114.22) (end 71 114.22) (width 0.25) (layer "F.Cu") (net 46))
 (segment (start 55.245 98.745) (end 65.725 98.745) (width 0.25) (layer "F.Cu") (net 46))
 (segment (start 92.71 91.87) (end 92.71 93.98) (width 0.25) (layer "F.Cu") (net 55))
 (segment (start 129.54 92.71) (end 129.54 95.25) (width 0.25) (layer "F.Cu") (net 55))
 (segment (start 129.54 95.25) (end 128.27 96.52) (width 0.25) (layer "F.Cu") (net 55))
 (segment (start 92.71 93.98) (end 93.98 95.25) (width 0.25) (layer "F.Cu") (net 55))
 (segment (start 110.49 96.52) (end 109.22 95.25) (width 0.25) (layer "F.Cu") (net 55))
 (segment (start 102.87 95.25) (end 109.22 88.9) (width 0.25) (layer "F.Cu") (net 55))
 (segment (start 93.98 95.25) (end 102.87 95.25) (width 0.25) (layer "F.Cu") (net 55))
 (segment (start 128.27 96.52) (end 110.49 96.52) (width 0.25) (layer "F.Cu") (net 55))
 (via (at 109.22 95.25) (size 0.8) (drill 0.4) (layers "F.Cu" "B.Cu") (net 55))
 (via (at 109.22 88.9) (size 0.8) (drill 0.4) (layers "F.Cu" "B.Cu") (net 55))
 (segment (start 109.22 88.9) (end 109.22 95.25) (width 0.25) (layer "B.Cu") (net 55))
 (segment (start 123.3575 51.355) (end 127 54.9975) (width 0.25) (layer "F.Cu") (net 74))
 (segment (start 127 60.96) (end 124.46 63.5) (width 0.25) (layer "F.Cu") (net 74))
 (segment (start 127 54.9975) (end 127 60.96) (width 0.25) (layer "F.Cu") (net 74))
 (segment (start 116.86 62.55) (end 116.84 62.53) (width 0.25) (layer "F.Cu") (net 75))
 (segment (start 116.84 62.53) (end 116.84 65.04) (width 0.25) (layer "F.Cu") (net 75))
 (segment (start 122.585 62.55) (end 116.86 62.55) (width 0.25) (layer "F.Cu") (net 75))
 (segment (start 91.44 96.52) (end 104.14 96.52) (width 0.25) (layer "F.Cu") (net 44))
 (segment (start 116.19 66.04) (end 121.92 66.04) (width 0.25) (layer "F.Cu") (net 44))
 (segment (start 104.14 96.52) (end 116.84 83.82) (width 0.25) (layer "F.Cu") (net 44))
 (segment (start 88.9 101.17) (end 88.9 99.06) (width 0.25) (layer "F.Cu") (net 44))
 (segment (start 86.36 101.17) (end 87.63 101.17) (width 0.25) (layer "F.Cu") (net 44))
 (segment (start 58.42 88.9) (end 58.105 89.215) (width 0.25) (layer "F.Cu") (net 44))
 (segment (start 58.105 89.215) (end 55.245 89.215) (width 0.25) (layer "F.Cu") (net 44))
 (segment (start 86.36 101.17) (end 70.69 101.17) (width 0.25) (layer "F.Cu") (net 44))
 (segment (start 127 92.71) (end 115.57 92.71) (width 0.25) (layer "F.Cu") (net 44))
 (segment (start 88.9 99.06) (end 91.44 96.52) (width 0.25) (layer "F.Cu") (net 44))
 (segment (start 122.585 65.375) (end 122.585 64.45) (width 0.25) (layer "F.Cu") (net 44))
 (segment (start 115.19 65.04) (end 116.19 66.04) (width 0.25) (layer "F.Cu") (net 44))
 (segment (start 115.57 92.71) (end 111.76 88.9) (width 0.25) (layer "F.Cu") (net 44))
 (segment (start 121.92 66.04) (end 122.585 65.375) (width 0.25) (layer "F.Cu") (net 44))
 (segment (start 91.44 91.87) (end 91.44 96.52) (width 0.25) (layer "F.Cu") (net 44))
 (segment (start 116.84 83.82) (end 116.84 66.04) (width 0.25) (layer "F.Cu") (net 44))
 (segment (start 70.69 101.17) (end 58.42 88.9) (width 0.25) (layer "F.Cu") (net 44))
 (segment (start 88.9 101.17) (end 87.63 101.17) (width 0.25) (layer "F.Cu") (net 44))
 (segment (start 137.16 91.44) (end 135.89 90.17) (width 0.25) (layer "B.Cu") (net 44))
 (segment (start 137.16 92.71) (end 137.16 91.44) (width 0.25) (layer "B.Cu") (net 44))
 (segment (start 128.27 90.17) (end 127 91.44) (width 0.25) (layer "B.Cu") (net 44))
 (segment (start 127 91.44) (end 127 92.71) (width 0.25) (layer "B.Cu") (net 44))
 (segment (start 135.89 90.17) (end 128.27 90.17) (width 0.25) (layer "B.Cu") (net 44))
 (segment (start 111.76 82.98) (end 111.76 65.96) (width 0.25) (layer "F.Cu") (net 47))
 (segment (start 111.76 65.96) (end 115.19 62.53) (width 0.25) (layer "F.Cu") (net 47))
 (segment (start 102.87 91.87) (end 111.76 82.98) (width 0.25) (layer "F.Cu") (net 47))
 (segment (start 52.705 83.44) (end 51.435 82.17) (width 0.25) (layer "F.Cu") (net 3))
 (segment (start 52.705 89.215) (end 52.705 83.44) (width 0.25) (layer "F.Cu") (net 3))
 (segment (start 50.8 73.66) (end 50.8 81.535) (width 0.25) (layer "F.Cu") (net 3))
 (segment (start 50.8 81.535) (end 51.435 82.17) (width 0.25) (layer "F.Cu") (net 3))
 (segment (start 66.04 86.36) (end 63.5 83.82) (width 0.25) (layer "F.Cu") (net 8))
 (segment (start 87.63 90.17) (end 83.82 86.36) (width 0.25) (layer "F.Cu") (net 8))
 (segment (start 83.82 86.36) (end 66.04 86.36) (width 0.25) (layer "F.Cu") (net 8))
 (segment (start 63.5 83.82) (end 63.5 73.66) (width 0.25) (layer "F.Cu") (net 8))
 (segment (start 87.63 91.87) (end 87.63 90.17) (width 0.25) (layer "F.Cu") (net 8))
 (segment (start 69.85 85.09) (end 66.04 81.28) (width 0.25) (layer "F.Cu") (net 9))
 (segment (start 83.82 85.09) (end 69.85 85.09) (width 0.25) (layer "F.Cu") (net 9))
 (segment (start 88.9 90.17) (end 83.82 85.09) (width 0.25) (layer "F.Cu") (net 9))
 (segment (start 66.04 81.28) (end 66.04 73.66) (width 0.25) (layer "F.Cu") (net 9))
 (segment (start 88.9 91.87) (end 88.9 90.17) (width 0.25) (layer "F.Cu") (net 9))
 (segment (start 93.98 55.88) (end 93.98 53.34) (width 0.25) (layer "F.Cu") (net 25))
 (segment (start 106.68 53.34) (end 106.68 83.82) (width 0.25) (layer "F.Cu") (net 25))
 (segment (start 90.17 101.17) (end 90.17 101.596751) (width 0.25) (layer "F.Cu") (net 25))
 (segment (start 93.98 53.34) (end 96.52 50.8) (width 0.25) (layer "F.Cu") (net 25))
 (segment (start 90.17 101.596751) (end 95.253249 106.68) (width 0.25) (layer "F.Cu") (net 25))
 (segment (start 104.14 50.8) (end 106.68 53.34) (width 0.25) (layer "F.Cu") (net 25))
 (segment (start 95.253249 106.68) (end 106.68 106.68) (width 0.25) (layer "F.Cu") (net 25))
 (segment (start 96.52 50.8) (end 104.14 50.8) (width 0.25) (layer "F.Cu") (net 25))
 (via (at 106.68 106.68) (size 0.8) (drill 0.4) (layers "F.Cu" "B.Cu") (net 25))
 (via (at 106.68 83.82) (size 0.8) (drill 0.4) (layers "F.Cu" "B.Cu") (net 25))
 (segment (start 106.68 83.82) (end 106.68 106.68) (width 0.25) (layer "B.Cu") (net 25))
 (segment (start 52.705 101.22) (end 51.435 102.49) (width 0.25) (layer "F.Cu") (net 2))
 (segment (start 52.705 98.745) (end 52.705 101.22) (width 0.25) (layer "F.Cu") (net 2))
 (segment (start 107.95 83.82) (end 107.95 55.88) (width 0.25) (layer "F.Cu") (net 23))
 (via (at 107.95 55.88) (size 0.8) (drill 0.4) (layers "F.Cu" "B.Cu") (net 23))
 (via (at 107.95 83.82) (size 0.8) (drill 0.4) (layers "F.Cu" "B.Cu") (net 23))
 (segment (start 107.95 55.88) (end 99.06 55.88) (width 0.25) (layer "B.Cu") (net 23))
 (segment (start 139.7 92.71) (end 139.7 90.17) (width 0.25) (layer "B.Cu") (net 23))
 (segment (start 113.03 88.9) (end 107.95 83.82) (width 0.25) (layer "B.Cu") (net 23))
 (segment (start 139.7 90.17) (end 138.43 88.9) (width 0.25) (layer "B.Cu") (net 23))
 (segment (start 138.43 88.9) (end 113.03 88.9) (width 0.25) (layer "B.Cu") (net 23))
 (segment (start 137.16 57.15) (end 137.16 74.71) (width 0.25) (layer "F.Cu") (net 24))
 (via (at 137.16 57.15) (size 0.8) (drill 0.4) (layers "F.Cu" "B.Cu") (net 24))
 (segment (start 97.79 57.15) (end 137.16 57.15) (width 0.25) (layer "B.Cu") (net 24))
 (segment (start 96.52 55.88) (end 97.79 57.15) (width 0.25) (layer "B.Cu") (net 24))
 (segment (start 134.62 58.42) (end 134.62 74.71) (width 0.25) (layer "F.Cu") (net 26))
 (via (at 134.62 58.42) (size 0.8) (drill 0.4) (layers "F.Cu" "B.Cu") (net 26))
 (segment (start 91.44 55.88) (end 91.44 57.15) (width 0.25) (layer "B.Cu") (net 26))
 (segment (start 92.71 58.42) (end 134.62 58.42) (width 0.25) (layer "B.Cu") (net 26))
 (segment (start 91.44 57.15) (end 92.71 58.42) (width 0.25) (layer "B.Cu") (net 26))
 (segment (start 132.08 59.69) (end 132.08 74.71) (width 0.25) (layer "F.Cu") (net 27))
 (via (at 132.08 59.69) (size 0.8) (drill 0.4) (layers "F.Cu" "B.Cu") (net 27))
 (segment (start 88.9 58.42) (end 90.17 59.69) (width 0.25) (layer "B.Cu") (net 27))
 (segment (start 88.9 55.88) (end 88.9 58.42) (width 0.25) (layer "B.Cu") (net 27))
 (segment (start 90.17 59.69) (end 132.08 59.69) (width 0.25) (layer "B.Cu") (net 27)))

